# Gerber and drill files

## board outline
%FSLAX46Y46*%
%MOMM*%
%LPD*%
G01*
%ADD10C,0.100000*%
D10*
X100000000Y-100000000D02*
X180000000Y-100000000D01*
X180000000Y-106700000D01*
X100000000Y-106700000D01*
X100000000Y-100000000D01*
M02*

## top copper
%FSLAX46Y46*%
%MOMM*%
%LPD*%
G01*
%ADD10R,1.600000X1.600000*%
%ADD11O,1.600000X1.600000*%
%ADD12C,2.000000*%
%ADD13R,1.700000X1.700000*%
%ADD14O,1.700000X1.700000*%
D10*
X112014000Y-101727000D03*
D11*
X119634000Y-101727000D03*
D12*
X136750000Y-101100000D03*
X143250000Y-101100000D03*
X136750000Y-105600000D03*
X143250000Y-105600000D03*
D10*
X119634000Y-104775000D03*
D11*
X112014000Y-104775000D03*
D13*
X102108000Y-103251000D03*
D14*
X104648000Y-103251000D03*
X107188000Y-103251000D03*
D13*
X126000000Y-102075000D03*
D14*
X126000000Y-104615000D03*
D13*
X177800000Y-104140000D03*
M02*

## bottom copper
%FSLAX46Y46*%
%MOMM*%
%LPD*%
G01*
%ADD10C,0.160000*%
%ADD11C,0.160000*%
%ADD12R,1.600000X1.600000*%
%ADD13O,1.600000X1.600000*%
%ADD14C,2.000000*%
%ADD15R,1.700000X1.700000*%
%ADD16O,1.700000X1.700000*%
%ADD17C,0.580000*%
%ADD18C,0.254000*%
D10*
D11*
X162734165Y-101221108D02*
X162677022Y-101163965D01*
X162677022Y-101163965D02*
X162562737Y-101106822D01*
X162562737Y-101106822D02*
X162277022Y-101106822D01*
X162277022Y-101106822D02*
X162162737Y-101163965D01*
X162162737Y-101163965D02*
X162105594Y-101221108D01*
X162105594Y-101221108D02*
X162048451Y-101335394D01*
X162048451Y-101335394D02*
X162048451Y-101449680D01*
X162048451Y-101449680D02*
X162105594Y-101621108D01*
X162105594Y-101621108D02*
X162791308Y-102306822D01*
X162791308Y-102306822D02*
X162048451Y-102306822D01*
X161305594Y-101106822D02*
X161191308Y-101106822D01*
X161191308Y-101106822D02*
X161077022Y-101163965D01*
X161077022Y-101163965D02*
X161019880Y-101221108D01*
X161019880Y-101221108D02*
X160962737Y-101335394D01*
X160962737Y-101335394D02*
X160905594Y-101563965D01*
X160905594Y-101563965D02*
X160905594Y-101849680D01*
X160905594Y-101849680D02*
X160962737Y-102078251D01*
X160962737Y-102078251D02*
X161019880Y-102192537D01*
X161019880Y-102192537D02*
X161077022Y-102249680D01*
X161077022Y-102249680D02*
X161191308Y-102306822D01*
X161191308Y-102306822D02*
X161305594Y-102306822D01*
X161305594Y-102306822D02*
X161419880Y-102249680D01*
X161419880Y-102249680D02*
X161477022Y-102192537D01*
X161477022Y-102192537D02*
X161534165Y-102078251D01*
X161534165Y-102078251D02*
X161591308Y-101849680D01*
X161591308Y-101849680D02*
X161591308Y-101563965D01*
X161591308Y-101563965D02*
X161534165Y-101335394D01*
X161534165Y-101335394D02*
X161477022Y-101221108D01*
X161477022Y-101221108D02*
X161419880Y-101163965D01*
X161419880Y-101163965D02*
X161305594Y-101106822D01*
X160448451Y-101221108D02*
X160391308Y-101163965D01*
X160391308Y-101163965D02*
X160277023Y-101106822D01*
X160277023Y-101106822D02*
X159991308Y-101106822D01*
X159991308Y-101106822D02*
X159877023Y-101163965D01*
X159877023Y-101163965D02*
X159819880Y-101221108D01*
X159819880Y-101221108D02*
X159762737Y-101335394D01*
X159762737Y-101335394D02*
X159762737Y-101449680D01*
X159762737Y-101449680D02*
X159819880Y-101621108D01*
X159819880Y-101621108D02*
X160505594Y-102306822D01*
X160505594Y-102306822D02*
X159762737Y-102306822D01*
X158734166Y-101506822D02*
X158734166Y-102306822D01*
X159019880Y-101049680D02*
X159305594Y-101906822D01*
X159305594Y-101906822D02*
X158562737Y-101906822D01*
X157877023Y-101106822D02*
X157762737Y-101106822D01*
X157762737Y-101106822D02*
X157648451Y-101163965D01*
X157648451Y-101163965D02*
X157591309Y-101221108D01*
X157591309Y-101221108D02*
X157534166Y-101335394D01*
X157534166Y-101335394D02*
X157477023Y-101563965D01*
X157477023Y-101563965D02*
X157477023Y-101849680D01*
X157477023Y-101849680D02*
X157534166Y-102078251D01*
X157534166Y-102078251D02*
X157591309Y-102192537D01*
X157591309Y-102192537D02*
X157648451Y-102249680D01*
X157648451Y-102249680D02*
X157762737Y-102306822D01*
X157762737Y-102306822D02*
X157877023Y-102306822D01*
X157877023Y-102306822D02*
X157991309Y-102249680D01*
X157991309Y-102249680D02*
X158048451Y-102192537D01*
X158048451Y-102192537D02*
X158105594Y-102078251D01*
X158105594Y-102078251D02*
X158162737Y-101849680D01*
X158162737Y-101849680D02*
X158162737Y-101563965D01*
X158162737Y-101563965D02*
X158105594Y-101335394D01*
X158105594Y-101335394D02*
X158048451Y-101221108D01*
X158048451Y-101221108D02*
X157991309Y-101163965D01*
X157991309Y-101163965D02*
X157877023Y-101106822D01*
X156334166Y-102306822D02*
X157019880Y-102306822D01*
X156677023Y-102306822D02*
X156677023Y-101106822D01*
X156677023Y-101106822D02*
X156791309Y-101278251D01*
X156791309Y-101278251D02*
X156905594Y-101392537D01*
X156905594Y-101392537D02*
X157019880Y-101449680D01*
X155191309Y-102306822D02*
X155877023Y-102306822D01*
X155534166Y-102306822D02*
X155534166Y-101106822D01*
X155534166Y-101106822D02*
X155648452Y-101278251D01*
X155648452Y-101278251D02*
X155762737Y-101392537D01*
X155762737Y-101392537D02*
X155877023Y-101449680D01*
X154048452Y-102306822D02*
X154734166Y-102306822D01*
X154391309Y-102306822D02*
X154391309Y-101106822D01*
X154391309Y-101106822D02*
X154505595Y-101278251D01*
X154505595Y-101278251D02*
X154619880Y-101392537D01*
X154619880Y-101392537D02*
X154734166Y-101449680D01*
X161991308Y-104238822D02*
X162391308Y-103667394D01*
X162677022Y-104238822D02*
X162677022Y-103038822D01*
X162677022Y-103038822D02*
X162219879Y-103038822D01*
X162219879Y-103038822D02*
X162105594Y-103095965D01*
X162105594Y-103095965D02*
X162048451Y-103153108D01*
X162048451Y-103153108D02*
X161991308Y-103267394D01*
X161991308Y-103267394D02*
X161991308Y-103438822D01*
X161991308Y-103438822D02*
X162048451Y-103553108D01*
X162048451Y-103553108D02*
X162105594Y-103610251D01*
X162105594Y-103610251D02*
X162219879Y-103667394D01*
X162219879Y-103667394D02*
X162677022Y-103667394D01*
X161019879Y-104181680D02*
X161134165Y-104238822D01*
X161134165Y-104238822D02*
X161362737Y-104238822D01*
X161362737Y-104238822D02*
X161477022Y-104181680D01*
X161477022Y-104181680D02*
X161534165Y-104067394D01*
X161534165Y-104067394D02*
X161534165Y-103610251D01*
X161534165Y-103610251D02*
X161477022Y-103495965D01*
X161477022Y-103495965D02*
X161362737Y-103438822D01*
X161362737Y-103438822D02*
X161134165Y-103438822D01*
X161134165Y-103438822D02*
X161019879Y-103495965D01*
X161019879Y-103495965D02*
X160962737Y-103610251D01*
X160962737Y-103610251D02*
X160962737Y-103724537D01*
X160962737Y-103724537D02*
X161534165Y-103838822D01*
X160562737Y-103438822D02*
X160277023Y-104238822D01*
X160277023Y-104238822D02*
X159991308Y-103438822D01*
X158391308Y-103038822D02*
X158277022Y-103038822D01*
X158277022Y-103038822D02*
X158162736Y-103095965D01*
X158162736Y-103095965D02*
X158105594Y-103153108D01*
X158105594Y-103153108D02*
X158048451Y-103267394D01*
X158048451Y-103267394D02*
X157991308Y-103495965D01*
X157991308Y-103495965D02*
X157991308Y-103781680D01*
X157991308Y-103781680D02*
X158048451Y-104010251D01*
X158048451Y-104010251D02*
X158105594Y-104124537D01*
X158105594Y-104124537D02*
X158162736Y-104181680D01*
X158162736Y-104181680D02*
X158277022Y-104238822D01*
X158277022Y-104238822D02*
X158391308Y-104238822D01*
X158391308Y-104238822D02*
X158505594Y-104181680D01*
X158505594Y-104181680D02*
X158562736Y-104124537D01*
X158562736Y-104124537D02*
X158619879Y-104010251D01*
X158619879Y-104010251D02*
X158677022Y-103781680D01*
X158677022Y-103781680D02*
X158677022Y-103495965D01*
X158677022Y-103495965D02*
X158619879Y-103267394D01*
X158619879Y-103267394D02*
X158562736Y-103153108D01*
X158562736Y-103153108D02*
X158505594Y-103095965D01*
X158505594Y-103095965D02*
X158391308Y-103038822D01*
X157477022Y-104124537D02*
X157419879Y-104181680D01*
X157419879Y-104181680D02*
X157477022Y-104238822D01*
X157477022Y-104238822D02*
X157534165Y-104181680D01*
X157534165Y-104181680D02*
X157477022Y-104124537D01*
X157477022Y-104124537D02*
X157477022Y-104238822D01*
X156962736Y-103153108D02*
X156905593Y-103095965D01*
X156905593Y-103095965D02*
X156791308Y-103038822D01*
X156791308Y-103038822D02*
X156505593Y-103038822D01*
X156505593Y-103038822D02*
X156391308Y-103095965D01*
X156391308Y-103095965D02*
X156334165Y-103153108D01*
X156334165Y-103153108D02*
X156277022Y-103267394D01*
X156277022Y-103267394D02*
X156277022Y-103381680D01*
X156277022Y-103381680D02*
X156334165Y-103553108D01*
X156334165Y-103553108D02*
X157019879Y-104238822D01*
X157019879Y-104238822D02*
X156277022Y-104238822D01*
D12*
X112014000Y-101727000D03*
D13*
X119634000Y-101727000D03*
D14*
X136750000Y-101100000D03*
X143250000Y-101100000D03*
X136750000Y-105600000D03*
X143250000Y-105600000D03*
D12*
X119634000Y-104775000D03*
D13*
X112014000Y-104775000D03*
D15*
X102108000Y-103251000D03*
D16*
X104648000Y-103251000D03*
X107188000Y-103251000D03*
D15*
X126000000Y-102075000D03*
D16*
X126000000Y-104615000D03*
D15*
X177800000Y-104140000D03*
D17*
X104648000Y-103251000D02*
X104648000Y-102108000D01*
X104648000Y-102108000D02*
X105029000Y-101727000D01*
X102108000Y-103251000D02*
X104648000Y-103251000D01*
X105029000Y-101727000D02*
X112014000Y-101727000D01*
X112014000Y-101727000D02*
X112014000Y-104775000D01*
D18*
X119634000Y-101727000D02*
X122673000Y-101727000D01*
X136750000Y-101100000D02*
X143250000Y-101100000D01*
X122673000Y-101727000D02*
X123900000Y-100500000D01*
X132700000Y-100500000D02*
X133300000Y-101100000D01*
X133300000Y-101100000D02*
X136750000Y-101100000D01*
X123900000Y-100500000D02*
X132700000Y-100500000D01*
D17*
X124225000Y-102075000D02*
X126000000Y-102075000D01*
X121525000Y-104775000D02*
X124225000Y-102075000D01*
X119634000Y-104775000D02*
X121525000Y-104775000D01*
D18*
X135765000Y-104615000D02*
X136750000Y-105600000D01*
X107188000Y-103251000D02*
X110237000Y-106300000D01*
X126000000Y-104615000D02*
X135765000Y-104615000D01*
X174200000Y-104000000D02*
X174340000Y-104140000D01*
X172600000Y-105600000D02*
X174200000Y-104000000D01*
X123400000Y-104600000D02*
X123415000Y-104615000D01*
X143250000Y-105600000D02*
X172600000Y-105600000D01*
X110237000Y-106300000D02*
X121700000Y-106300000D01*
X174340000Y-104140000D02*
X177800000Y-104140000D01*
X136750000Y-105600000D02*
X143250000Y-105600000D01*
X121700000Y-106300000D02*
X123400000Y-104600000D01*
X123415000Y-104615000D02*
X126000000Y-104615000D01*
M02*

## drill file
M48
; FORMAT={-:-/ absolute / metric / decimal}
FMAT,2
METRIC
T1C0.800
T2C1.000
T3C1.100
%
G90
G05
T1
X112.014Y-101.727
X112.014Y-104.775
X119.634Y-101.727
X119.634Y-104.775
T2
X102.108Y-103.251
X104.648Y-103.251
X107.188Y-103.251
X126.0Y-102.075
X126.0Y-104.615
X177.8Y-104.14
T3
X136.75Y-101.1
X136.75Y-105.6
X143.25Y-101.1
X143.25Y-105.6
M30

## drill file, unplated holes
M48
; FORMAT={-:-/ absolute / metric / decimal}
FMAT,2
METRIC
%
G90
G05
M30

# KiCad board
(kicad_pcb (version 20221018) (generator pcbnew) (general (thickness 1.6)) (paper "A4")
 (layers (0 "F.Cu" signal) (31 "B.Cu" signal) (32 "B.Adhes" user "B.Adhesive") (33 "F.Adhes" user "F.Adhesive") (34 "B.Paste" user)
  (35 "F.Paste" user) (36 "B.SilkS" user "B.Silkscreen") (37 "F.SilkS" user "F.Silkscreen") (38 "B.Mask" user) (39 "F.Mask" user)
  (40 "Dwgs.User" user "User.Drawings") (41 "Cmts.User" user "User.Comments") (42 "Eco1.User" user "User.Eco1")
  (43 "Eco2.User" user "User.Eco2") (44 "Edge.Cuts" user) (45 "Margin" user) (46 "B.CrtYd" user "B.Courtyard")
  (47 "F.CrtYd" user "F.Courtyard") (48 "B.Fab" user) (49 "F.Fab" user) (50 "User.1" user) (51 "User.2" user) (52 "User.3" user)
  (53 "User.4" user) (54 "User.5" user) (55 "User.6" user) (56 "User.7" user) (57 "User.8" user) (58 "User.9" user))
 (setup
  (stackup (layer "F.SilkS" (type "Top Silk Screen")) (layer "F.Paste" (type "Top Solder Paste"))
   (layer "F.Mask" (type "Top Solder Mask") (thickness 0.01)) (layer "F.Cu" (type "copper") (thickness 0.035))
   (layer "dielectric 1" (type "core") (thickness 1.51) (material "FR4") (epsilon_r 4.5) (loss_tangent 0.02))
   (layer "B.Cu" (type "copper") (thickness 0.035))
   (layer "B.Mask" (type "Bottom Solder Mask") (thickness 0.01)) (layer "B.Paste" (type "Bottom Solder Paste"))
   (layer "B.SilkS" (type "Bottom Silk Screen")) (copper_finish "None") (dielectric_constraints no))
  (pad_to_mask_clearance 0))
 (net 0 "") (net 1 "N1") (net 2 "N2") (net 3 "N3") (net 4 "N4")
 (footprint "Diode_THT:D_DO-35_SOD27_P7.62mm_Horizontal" (layer "F.Cu") (at 112.014 101.727)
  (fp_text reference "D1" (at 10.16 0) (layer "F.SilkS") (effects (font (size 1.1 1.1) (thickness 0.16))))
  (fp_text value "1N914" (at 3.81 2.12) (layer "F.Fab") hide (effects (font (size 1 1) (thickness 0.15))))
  (pad "1" thru_hole rect (at 0 0) (size 1.6 1.6) (drill 0.8) (layers "*.Cu" "*.Mask") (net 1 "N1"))
  (pad "2" thru_hole oval (at 7.62 0) (size 1.6 1.6) (drill 0.8) (layers "*.Cu" "*.Mask") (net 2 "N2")))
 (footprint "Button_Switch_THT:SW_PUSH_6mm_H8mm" (layer "F.Cu") (at 136.75 101.1)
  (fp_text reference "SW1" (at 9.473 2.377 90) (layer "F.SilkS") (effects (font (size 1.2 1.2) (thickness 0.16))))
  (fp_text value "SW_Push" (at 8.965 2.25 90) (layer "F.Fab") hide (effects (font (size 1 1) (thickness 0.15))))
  (pad "1" thru_hole circle (at 0 0 90) (size 2 2) (drill 1.1) (layers "*.Cu" "*.Mask") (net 2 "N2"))
  (pad "1" thru_hole circle (at 6.5 0 90) (size 2 2) (drill 1.1) (layers "*.Cu" "*.Mask") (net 2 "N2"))
  (pad "2" thru_hole circle (at 0 4.5 90) (size 2 2) (drill 1.1) (layers "*.Cu" "*.Mask") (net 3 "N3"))
  (pad "2" thru_hole circle (at 6.5 4.5 90) (size 2 2) (drill 1.1) (layers "*.Cu" "*.Mask") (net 3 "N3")))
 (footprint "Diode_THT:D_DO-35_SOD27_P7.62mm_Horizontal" (layer "F.Cu") (at 119.634 104.775 180)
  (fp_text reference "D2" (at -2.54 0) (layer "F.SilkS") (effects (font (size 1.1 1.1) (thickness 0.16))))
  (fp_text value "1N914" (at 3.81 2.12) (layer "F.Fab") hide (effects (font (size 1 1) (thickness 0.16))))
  (pad "1" thru_hole rect (at 0 0 180) (size 1.6 1.6) (drill 0.8) (layers "*.Cu" "*.Mask") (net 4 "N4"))
  (pad "2" thru_hole oval (at 7.62 0 180) (size 1.6 1.6) (drill 0.8) (layers "*.Cu" "*.Mask") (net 1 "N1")))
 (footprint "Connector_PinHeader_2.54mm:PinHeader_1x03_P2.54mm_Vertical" (layer "F.Cu") (at 102.108 103.251 90)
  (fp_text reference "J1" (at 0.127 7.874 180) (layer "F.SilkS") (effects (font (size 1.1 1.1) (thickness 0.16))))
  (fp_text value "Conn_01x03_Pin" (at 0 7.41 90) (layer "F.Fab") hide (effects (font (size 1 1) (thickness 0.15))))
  (pad "1" thru_hole rect (at 0 0 90) (size 1.7 1.7) (drill 1) (layers "*.Cu" "*.Mask") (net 1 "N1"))
  (pad "2" thru_hole oval (at 0 2.54 90) (size 1.7 1.7) (drill 1) (layers "*.Cu" "*.Mask") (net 1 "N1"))
  (pad "3" thru_hole oval (at 0 5.08 90) (size 1.7 1.7) (drill 1) (layers "*.Cu" "*.Mask") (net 3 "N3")))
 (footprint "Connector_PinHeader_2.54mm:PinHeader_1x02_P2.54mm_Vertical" (layer "F.Cu") (at 126 102.075)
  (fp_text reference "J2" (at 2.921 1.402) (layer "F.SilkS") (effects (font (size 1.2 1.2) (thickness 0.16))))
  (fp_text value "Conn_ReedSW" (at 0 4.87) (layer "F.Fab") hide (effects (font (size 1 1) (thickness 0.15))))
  (pad "1" thru_hole rect (at 0 0) (size 1.7 1.7) (drill 1) (layers "*.Cu" "*.Mask") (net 4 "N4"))
  (pad "2" thru_hole oval (at 0 2.54) (size 1.7 1.7) (drill 1) (layers "*.Cu" "*.Mask") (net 3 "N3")))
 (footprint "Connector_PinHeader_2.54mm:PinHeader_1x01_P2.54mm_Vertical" (layer "F.Cu") (at 177.8 104.14)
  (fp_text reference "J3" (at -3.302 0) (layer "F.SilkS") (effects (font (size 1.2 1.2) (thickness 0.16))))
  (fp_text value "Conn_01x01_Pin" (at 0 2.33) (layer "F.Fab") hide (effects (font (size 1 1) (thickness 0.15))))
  (pad "1" thru_hole rect (at 0 0) (size 1.7 1.7) (drill 1) (layers "*.Cu" "*.Mask") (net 3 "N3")))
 (gr_rect (start 100 100) (end 180 106.7) (stroke (width 0.1) (type solid)) (fill none) (layer "Edge.Cuts"))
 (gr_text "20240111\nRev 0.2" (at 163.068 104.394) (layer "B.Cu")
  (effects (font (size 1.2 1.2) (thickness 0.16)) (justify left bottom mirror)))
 (segment (start 104.648 103.251) (end 104.648 102.108) (width 0.58) (layer "B.Cu") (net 1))
 (segment (start 104.648 102.108) (end 105.029 101.727) (width 0.58) (layer "B.Cu") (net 1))
 (segment (start 102.108 103.251) (end 104.648 103.251) (width 0.58) (layer "B.Cu") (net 1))
 (segment (start 105.029 101.727) (end 112.014 101.727) (width 0.58) (layer "B.Cu") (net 1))
 (segment (start 112.014 101.727) (end 112.014 104.775) (width 0.58) (layer "B.Cu") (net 1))
 (segment (start 119.634 101.727) (end 122.673 101.727) (width 0.254) (layer "B.Cu") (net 2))
 (segment (start 136.75 101.1) (end 143.25 101.1) (width 0.254) (layer "B.Cu") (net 2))
 (segment (start 122.673 101.727) (end 123.9 100.5) (width 0.254) (layer "B.Cu") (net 2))
 (segment (start 132.7 100.5) (end 133.3 101.1) (width 0.254) (layer "B.Cu") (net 2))
 (segment (start 133.3 101.1) (end 136.75 101.1) (width 0.254) (layer "B.Cu") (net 2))
 (segment (start 123.9 100.5) (end 132.7 100.5) (width 0.254) (layer "B.Cu") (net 2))
 (segment (start 124.225 102.075) (end 126 102.075) (width 0.58) (layer "B.Cu") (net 4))
 (segment (start 121.525 104.775) (end 124.225 102.075) (width 0.58) (layer "B.Cu") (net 4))
 (segment (start 119.634 104.775) (end 121.525 104.775) (width 0.58) (layer "B.Cu") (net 4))
 (segment (start 135.765 104.615) (end 136.75 105.6) (width 0.254) (layer "B.Cu") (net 3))
 (segment (start 107.188 103.251) (end 110.237 106.3) (width 0.254) (layer "B.Cu") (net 3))
 (segment (start 126 104.615) (end 135.765 104.615) (width 0.254) (layer "B.Cu") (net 3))
 (segment (start 174.2 104) (end 174.34 104.14) (width 0.254) (layer "B.Cu") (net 3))
 (segment (start 172.6 105.6) (end 174.2 104) (width 0.254) (layer "B.Cu") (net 3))
 (segment (start 123.4 104.6) (end 123.415 104.615) (width 0.254) (layer "B.Cu") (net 3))
 (segment (start 143.25 105.6) (end 172.6 105.6) (width 0.254) (layer "B.Cu") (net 3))
 (segment (start 110.237 106.3) (end 121.7 106.3) (width 0.254) (layer "B.Cu") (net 3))
 (segment (start 174.34 104.14) (end 177.8 104.14) (width 0.254) (layer "B.Cu") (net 3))
 (segment (start 136.75 105.6) (end 143.25 105.6) (width 0.254) (layer "B.Cu") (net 3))
 (segment (start 121.7 106.3) (end 123.4 104.6) (width 0.254) (layer "B.Cu") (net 3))
 (segment (start 123.415 104.615) (end 126 104.615) (width 0.254) (layer "B.Cu") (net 3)))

